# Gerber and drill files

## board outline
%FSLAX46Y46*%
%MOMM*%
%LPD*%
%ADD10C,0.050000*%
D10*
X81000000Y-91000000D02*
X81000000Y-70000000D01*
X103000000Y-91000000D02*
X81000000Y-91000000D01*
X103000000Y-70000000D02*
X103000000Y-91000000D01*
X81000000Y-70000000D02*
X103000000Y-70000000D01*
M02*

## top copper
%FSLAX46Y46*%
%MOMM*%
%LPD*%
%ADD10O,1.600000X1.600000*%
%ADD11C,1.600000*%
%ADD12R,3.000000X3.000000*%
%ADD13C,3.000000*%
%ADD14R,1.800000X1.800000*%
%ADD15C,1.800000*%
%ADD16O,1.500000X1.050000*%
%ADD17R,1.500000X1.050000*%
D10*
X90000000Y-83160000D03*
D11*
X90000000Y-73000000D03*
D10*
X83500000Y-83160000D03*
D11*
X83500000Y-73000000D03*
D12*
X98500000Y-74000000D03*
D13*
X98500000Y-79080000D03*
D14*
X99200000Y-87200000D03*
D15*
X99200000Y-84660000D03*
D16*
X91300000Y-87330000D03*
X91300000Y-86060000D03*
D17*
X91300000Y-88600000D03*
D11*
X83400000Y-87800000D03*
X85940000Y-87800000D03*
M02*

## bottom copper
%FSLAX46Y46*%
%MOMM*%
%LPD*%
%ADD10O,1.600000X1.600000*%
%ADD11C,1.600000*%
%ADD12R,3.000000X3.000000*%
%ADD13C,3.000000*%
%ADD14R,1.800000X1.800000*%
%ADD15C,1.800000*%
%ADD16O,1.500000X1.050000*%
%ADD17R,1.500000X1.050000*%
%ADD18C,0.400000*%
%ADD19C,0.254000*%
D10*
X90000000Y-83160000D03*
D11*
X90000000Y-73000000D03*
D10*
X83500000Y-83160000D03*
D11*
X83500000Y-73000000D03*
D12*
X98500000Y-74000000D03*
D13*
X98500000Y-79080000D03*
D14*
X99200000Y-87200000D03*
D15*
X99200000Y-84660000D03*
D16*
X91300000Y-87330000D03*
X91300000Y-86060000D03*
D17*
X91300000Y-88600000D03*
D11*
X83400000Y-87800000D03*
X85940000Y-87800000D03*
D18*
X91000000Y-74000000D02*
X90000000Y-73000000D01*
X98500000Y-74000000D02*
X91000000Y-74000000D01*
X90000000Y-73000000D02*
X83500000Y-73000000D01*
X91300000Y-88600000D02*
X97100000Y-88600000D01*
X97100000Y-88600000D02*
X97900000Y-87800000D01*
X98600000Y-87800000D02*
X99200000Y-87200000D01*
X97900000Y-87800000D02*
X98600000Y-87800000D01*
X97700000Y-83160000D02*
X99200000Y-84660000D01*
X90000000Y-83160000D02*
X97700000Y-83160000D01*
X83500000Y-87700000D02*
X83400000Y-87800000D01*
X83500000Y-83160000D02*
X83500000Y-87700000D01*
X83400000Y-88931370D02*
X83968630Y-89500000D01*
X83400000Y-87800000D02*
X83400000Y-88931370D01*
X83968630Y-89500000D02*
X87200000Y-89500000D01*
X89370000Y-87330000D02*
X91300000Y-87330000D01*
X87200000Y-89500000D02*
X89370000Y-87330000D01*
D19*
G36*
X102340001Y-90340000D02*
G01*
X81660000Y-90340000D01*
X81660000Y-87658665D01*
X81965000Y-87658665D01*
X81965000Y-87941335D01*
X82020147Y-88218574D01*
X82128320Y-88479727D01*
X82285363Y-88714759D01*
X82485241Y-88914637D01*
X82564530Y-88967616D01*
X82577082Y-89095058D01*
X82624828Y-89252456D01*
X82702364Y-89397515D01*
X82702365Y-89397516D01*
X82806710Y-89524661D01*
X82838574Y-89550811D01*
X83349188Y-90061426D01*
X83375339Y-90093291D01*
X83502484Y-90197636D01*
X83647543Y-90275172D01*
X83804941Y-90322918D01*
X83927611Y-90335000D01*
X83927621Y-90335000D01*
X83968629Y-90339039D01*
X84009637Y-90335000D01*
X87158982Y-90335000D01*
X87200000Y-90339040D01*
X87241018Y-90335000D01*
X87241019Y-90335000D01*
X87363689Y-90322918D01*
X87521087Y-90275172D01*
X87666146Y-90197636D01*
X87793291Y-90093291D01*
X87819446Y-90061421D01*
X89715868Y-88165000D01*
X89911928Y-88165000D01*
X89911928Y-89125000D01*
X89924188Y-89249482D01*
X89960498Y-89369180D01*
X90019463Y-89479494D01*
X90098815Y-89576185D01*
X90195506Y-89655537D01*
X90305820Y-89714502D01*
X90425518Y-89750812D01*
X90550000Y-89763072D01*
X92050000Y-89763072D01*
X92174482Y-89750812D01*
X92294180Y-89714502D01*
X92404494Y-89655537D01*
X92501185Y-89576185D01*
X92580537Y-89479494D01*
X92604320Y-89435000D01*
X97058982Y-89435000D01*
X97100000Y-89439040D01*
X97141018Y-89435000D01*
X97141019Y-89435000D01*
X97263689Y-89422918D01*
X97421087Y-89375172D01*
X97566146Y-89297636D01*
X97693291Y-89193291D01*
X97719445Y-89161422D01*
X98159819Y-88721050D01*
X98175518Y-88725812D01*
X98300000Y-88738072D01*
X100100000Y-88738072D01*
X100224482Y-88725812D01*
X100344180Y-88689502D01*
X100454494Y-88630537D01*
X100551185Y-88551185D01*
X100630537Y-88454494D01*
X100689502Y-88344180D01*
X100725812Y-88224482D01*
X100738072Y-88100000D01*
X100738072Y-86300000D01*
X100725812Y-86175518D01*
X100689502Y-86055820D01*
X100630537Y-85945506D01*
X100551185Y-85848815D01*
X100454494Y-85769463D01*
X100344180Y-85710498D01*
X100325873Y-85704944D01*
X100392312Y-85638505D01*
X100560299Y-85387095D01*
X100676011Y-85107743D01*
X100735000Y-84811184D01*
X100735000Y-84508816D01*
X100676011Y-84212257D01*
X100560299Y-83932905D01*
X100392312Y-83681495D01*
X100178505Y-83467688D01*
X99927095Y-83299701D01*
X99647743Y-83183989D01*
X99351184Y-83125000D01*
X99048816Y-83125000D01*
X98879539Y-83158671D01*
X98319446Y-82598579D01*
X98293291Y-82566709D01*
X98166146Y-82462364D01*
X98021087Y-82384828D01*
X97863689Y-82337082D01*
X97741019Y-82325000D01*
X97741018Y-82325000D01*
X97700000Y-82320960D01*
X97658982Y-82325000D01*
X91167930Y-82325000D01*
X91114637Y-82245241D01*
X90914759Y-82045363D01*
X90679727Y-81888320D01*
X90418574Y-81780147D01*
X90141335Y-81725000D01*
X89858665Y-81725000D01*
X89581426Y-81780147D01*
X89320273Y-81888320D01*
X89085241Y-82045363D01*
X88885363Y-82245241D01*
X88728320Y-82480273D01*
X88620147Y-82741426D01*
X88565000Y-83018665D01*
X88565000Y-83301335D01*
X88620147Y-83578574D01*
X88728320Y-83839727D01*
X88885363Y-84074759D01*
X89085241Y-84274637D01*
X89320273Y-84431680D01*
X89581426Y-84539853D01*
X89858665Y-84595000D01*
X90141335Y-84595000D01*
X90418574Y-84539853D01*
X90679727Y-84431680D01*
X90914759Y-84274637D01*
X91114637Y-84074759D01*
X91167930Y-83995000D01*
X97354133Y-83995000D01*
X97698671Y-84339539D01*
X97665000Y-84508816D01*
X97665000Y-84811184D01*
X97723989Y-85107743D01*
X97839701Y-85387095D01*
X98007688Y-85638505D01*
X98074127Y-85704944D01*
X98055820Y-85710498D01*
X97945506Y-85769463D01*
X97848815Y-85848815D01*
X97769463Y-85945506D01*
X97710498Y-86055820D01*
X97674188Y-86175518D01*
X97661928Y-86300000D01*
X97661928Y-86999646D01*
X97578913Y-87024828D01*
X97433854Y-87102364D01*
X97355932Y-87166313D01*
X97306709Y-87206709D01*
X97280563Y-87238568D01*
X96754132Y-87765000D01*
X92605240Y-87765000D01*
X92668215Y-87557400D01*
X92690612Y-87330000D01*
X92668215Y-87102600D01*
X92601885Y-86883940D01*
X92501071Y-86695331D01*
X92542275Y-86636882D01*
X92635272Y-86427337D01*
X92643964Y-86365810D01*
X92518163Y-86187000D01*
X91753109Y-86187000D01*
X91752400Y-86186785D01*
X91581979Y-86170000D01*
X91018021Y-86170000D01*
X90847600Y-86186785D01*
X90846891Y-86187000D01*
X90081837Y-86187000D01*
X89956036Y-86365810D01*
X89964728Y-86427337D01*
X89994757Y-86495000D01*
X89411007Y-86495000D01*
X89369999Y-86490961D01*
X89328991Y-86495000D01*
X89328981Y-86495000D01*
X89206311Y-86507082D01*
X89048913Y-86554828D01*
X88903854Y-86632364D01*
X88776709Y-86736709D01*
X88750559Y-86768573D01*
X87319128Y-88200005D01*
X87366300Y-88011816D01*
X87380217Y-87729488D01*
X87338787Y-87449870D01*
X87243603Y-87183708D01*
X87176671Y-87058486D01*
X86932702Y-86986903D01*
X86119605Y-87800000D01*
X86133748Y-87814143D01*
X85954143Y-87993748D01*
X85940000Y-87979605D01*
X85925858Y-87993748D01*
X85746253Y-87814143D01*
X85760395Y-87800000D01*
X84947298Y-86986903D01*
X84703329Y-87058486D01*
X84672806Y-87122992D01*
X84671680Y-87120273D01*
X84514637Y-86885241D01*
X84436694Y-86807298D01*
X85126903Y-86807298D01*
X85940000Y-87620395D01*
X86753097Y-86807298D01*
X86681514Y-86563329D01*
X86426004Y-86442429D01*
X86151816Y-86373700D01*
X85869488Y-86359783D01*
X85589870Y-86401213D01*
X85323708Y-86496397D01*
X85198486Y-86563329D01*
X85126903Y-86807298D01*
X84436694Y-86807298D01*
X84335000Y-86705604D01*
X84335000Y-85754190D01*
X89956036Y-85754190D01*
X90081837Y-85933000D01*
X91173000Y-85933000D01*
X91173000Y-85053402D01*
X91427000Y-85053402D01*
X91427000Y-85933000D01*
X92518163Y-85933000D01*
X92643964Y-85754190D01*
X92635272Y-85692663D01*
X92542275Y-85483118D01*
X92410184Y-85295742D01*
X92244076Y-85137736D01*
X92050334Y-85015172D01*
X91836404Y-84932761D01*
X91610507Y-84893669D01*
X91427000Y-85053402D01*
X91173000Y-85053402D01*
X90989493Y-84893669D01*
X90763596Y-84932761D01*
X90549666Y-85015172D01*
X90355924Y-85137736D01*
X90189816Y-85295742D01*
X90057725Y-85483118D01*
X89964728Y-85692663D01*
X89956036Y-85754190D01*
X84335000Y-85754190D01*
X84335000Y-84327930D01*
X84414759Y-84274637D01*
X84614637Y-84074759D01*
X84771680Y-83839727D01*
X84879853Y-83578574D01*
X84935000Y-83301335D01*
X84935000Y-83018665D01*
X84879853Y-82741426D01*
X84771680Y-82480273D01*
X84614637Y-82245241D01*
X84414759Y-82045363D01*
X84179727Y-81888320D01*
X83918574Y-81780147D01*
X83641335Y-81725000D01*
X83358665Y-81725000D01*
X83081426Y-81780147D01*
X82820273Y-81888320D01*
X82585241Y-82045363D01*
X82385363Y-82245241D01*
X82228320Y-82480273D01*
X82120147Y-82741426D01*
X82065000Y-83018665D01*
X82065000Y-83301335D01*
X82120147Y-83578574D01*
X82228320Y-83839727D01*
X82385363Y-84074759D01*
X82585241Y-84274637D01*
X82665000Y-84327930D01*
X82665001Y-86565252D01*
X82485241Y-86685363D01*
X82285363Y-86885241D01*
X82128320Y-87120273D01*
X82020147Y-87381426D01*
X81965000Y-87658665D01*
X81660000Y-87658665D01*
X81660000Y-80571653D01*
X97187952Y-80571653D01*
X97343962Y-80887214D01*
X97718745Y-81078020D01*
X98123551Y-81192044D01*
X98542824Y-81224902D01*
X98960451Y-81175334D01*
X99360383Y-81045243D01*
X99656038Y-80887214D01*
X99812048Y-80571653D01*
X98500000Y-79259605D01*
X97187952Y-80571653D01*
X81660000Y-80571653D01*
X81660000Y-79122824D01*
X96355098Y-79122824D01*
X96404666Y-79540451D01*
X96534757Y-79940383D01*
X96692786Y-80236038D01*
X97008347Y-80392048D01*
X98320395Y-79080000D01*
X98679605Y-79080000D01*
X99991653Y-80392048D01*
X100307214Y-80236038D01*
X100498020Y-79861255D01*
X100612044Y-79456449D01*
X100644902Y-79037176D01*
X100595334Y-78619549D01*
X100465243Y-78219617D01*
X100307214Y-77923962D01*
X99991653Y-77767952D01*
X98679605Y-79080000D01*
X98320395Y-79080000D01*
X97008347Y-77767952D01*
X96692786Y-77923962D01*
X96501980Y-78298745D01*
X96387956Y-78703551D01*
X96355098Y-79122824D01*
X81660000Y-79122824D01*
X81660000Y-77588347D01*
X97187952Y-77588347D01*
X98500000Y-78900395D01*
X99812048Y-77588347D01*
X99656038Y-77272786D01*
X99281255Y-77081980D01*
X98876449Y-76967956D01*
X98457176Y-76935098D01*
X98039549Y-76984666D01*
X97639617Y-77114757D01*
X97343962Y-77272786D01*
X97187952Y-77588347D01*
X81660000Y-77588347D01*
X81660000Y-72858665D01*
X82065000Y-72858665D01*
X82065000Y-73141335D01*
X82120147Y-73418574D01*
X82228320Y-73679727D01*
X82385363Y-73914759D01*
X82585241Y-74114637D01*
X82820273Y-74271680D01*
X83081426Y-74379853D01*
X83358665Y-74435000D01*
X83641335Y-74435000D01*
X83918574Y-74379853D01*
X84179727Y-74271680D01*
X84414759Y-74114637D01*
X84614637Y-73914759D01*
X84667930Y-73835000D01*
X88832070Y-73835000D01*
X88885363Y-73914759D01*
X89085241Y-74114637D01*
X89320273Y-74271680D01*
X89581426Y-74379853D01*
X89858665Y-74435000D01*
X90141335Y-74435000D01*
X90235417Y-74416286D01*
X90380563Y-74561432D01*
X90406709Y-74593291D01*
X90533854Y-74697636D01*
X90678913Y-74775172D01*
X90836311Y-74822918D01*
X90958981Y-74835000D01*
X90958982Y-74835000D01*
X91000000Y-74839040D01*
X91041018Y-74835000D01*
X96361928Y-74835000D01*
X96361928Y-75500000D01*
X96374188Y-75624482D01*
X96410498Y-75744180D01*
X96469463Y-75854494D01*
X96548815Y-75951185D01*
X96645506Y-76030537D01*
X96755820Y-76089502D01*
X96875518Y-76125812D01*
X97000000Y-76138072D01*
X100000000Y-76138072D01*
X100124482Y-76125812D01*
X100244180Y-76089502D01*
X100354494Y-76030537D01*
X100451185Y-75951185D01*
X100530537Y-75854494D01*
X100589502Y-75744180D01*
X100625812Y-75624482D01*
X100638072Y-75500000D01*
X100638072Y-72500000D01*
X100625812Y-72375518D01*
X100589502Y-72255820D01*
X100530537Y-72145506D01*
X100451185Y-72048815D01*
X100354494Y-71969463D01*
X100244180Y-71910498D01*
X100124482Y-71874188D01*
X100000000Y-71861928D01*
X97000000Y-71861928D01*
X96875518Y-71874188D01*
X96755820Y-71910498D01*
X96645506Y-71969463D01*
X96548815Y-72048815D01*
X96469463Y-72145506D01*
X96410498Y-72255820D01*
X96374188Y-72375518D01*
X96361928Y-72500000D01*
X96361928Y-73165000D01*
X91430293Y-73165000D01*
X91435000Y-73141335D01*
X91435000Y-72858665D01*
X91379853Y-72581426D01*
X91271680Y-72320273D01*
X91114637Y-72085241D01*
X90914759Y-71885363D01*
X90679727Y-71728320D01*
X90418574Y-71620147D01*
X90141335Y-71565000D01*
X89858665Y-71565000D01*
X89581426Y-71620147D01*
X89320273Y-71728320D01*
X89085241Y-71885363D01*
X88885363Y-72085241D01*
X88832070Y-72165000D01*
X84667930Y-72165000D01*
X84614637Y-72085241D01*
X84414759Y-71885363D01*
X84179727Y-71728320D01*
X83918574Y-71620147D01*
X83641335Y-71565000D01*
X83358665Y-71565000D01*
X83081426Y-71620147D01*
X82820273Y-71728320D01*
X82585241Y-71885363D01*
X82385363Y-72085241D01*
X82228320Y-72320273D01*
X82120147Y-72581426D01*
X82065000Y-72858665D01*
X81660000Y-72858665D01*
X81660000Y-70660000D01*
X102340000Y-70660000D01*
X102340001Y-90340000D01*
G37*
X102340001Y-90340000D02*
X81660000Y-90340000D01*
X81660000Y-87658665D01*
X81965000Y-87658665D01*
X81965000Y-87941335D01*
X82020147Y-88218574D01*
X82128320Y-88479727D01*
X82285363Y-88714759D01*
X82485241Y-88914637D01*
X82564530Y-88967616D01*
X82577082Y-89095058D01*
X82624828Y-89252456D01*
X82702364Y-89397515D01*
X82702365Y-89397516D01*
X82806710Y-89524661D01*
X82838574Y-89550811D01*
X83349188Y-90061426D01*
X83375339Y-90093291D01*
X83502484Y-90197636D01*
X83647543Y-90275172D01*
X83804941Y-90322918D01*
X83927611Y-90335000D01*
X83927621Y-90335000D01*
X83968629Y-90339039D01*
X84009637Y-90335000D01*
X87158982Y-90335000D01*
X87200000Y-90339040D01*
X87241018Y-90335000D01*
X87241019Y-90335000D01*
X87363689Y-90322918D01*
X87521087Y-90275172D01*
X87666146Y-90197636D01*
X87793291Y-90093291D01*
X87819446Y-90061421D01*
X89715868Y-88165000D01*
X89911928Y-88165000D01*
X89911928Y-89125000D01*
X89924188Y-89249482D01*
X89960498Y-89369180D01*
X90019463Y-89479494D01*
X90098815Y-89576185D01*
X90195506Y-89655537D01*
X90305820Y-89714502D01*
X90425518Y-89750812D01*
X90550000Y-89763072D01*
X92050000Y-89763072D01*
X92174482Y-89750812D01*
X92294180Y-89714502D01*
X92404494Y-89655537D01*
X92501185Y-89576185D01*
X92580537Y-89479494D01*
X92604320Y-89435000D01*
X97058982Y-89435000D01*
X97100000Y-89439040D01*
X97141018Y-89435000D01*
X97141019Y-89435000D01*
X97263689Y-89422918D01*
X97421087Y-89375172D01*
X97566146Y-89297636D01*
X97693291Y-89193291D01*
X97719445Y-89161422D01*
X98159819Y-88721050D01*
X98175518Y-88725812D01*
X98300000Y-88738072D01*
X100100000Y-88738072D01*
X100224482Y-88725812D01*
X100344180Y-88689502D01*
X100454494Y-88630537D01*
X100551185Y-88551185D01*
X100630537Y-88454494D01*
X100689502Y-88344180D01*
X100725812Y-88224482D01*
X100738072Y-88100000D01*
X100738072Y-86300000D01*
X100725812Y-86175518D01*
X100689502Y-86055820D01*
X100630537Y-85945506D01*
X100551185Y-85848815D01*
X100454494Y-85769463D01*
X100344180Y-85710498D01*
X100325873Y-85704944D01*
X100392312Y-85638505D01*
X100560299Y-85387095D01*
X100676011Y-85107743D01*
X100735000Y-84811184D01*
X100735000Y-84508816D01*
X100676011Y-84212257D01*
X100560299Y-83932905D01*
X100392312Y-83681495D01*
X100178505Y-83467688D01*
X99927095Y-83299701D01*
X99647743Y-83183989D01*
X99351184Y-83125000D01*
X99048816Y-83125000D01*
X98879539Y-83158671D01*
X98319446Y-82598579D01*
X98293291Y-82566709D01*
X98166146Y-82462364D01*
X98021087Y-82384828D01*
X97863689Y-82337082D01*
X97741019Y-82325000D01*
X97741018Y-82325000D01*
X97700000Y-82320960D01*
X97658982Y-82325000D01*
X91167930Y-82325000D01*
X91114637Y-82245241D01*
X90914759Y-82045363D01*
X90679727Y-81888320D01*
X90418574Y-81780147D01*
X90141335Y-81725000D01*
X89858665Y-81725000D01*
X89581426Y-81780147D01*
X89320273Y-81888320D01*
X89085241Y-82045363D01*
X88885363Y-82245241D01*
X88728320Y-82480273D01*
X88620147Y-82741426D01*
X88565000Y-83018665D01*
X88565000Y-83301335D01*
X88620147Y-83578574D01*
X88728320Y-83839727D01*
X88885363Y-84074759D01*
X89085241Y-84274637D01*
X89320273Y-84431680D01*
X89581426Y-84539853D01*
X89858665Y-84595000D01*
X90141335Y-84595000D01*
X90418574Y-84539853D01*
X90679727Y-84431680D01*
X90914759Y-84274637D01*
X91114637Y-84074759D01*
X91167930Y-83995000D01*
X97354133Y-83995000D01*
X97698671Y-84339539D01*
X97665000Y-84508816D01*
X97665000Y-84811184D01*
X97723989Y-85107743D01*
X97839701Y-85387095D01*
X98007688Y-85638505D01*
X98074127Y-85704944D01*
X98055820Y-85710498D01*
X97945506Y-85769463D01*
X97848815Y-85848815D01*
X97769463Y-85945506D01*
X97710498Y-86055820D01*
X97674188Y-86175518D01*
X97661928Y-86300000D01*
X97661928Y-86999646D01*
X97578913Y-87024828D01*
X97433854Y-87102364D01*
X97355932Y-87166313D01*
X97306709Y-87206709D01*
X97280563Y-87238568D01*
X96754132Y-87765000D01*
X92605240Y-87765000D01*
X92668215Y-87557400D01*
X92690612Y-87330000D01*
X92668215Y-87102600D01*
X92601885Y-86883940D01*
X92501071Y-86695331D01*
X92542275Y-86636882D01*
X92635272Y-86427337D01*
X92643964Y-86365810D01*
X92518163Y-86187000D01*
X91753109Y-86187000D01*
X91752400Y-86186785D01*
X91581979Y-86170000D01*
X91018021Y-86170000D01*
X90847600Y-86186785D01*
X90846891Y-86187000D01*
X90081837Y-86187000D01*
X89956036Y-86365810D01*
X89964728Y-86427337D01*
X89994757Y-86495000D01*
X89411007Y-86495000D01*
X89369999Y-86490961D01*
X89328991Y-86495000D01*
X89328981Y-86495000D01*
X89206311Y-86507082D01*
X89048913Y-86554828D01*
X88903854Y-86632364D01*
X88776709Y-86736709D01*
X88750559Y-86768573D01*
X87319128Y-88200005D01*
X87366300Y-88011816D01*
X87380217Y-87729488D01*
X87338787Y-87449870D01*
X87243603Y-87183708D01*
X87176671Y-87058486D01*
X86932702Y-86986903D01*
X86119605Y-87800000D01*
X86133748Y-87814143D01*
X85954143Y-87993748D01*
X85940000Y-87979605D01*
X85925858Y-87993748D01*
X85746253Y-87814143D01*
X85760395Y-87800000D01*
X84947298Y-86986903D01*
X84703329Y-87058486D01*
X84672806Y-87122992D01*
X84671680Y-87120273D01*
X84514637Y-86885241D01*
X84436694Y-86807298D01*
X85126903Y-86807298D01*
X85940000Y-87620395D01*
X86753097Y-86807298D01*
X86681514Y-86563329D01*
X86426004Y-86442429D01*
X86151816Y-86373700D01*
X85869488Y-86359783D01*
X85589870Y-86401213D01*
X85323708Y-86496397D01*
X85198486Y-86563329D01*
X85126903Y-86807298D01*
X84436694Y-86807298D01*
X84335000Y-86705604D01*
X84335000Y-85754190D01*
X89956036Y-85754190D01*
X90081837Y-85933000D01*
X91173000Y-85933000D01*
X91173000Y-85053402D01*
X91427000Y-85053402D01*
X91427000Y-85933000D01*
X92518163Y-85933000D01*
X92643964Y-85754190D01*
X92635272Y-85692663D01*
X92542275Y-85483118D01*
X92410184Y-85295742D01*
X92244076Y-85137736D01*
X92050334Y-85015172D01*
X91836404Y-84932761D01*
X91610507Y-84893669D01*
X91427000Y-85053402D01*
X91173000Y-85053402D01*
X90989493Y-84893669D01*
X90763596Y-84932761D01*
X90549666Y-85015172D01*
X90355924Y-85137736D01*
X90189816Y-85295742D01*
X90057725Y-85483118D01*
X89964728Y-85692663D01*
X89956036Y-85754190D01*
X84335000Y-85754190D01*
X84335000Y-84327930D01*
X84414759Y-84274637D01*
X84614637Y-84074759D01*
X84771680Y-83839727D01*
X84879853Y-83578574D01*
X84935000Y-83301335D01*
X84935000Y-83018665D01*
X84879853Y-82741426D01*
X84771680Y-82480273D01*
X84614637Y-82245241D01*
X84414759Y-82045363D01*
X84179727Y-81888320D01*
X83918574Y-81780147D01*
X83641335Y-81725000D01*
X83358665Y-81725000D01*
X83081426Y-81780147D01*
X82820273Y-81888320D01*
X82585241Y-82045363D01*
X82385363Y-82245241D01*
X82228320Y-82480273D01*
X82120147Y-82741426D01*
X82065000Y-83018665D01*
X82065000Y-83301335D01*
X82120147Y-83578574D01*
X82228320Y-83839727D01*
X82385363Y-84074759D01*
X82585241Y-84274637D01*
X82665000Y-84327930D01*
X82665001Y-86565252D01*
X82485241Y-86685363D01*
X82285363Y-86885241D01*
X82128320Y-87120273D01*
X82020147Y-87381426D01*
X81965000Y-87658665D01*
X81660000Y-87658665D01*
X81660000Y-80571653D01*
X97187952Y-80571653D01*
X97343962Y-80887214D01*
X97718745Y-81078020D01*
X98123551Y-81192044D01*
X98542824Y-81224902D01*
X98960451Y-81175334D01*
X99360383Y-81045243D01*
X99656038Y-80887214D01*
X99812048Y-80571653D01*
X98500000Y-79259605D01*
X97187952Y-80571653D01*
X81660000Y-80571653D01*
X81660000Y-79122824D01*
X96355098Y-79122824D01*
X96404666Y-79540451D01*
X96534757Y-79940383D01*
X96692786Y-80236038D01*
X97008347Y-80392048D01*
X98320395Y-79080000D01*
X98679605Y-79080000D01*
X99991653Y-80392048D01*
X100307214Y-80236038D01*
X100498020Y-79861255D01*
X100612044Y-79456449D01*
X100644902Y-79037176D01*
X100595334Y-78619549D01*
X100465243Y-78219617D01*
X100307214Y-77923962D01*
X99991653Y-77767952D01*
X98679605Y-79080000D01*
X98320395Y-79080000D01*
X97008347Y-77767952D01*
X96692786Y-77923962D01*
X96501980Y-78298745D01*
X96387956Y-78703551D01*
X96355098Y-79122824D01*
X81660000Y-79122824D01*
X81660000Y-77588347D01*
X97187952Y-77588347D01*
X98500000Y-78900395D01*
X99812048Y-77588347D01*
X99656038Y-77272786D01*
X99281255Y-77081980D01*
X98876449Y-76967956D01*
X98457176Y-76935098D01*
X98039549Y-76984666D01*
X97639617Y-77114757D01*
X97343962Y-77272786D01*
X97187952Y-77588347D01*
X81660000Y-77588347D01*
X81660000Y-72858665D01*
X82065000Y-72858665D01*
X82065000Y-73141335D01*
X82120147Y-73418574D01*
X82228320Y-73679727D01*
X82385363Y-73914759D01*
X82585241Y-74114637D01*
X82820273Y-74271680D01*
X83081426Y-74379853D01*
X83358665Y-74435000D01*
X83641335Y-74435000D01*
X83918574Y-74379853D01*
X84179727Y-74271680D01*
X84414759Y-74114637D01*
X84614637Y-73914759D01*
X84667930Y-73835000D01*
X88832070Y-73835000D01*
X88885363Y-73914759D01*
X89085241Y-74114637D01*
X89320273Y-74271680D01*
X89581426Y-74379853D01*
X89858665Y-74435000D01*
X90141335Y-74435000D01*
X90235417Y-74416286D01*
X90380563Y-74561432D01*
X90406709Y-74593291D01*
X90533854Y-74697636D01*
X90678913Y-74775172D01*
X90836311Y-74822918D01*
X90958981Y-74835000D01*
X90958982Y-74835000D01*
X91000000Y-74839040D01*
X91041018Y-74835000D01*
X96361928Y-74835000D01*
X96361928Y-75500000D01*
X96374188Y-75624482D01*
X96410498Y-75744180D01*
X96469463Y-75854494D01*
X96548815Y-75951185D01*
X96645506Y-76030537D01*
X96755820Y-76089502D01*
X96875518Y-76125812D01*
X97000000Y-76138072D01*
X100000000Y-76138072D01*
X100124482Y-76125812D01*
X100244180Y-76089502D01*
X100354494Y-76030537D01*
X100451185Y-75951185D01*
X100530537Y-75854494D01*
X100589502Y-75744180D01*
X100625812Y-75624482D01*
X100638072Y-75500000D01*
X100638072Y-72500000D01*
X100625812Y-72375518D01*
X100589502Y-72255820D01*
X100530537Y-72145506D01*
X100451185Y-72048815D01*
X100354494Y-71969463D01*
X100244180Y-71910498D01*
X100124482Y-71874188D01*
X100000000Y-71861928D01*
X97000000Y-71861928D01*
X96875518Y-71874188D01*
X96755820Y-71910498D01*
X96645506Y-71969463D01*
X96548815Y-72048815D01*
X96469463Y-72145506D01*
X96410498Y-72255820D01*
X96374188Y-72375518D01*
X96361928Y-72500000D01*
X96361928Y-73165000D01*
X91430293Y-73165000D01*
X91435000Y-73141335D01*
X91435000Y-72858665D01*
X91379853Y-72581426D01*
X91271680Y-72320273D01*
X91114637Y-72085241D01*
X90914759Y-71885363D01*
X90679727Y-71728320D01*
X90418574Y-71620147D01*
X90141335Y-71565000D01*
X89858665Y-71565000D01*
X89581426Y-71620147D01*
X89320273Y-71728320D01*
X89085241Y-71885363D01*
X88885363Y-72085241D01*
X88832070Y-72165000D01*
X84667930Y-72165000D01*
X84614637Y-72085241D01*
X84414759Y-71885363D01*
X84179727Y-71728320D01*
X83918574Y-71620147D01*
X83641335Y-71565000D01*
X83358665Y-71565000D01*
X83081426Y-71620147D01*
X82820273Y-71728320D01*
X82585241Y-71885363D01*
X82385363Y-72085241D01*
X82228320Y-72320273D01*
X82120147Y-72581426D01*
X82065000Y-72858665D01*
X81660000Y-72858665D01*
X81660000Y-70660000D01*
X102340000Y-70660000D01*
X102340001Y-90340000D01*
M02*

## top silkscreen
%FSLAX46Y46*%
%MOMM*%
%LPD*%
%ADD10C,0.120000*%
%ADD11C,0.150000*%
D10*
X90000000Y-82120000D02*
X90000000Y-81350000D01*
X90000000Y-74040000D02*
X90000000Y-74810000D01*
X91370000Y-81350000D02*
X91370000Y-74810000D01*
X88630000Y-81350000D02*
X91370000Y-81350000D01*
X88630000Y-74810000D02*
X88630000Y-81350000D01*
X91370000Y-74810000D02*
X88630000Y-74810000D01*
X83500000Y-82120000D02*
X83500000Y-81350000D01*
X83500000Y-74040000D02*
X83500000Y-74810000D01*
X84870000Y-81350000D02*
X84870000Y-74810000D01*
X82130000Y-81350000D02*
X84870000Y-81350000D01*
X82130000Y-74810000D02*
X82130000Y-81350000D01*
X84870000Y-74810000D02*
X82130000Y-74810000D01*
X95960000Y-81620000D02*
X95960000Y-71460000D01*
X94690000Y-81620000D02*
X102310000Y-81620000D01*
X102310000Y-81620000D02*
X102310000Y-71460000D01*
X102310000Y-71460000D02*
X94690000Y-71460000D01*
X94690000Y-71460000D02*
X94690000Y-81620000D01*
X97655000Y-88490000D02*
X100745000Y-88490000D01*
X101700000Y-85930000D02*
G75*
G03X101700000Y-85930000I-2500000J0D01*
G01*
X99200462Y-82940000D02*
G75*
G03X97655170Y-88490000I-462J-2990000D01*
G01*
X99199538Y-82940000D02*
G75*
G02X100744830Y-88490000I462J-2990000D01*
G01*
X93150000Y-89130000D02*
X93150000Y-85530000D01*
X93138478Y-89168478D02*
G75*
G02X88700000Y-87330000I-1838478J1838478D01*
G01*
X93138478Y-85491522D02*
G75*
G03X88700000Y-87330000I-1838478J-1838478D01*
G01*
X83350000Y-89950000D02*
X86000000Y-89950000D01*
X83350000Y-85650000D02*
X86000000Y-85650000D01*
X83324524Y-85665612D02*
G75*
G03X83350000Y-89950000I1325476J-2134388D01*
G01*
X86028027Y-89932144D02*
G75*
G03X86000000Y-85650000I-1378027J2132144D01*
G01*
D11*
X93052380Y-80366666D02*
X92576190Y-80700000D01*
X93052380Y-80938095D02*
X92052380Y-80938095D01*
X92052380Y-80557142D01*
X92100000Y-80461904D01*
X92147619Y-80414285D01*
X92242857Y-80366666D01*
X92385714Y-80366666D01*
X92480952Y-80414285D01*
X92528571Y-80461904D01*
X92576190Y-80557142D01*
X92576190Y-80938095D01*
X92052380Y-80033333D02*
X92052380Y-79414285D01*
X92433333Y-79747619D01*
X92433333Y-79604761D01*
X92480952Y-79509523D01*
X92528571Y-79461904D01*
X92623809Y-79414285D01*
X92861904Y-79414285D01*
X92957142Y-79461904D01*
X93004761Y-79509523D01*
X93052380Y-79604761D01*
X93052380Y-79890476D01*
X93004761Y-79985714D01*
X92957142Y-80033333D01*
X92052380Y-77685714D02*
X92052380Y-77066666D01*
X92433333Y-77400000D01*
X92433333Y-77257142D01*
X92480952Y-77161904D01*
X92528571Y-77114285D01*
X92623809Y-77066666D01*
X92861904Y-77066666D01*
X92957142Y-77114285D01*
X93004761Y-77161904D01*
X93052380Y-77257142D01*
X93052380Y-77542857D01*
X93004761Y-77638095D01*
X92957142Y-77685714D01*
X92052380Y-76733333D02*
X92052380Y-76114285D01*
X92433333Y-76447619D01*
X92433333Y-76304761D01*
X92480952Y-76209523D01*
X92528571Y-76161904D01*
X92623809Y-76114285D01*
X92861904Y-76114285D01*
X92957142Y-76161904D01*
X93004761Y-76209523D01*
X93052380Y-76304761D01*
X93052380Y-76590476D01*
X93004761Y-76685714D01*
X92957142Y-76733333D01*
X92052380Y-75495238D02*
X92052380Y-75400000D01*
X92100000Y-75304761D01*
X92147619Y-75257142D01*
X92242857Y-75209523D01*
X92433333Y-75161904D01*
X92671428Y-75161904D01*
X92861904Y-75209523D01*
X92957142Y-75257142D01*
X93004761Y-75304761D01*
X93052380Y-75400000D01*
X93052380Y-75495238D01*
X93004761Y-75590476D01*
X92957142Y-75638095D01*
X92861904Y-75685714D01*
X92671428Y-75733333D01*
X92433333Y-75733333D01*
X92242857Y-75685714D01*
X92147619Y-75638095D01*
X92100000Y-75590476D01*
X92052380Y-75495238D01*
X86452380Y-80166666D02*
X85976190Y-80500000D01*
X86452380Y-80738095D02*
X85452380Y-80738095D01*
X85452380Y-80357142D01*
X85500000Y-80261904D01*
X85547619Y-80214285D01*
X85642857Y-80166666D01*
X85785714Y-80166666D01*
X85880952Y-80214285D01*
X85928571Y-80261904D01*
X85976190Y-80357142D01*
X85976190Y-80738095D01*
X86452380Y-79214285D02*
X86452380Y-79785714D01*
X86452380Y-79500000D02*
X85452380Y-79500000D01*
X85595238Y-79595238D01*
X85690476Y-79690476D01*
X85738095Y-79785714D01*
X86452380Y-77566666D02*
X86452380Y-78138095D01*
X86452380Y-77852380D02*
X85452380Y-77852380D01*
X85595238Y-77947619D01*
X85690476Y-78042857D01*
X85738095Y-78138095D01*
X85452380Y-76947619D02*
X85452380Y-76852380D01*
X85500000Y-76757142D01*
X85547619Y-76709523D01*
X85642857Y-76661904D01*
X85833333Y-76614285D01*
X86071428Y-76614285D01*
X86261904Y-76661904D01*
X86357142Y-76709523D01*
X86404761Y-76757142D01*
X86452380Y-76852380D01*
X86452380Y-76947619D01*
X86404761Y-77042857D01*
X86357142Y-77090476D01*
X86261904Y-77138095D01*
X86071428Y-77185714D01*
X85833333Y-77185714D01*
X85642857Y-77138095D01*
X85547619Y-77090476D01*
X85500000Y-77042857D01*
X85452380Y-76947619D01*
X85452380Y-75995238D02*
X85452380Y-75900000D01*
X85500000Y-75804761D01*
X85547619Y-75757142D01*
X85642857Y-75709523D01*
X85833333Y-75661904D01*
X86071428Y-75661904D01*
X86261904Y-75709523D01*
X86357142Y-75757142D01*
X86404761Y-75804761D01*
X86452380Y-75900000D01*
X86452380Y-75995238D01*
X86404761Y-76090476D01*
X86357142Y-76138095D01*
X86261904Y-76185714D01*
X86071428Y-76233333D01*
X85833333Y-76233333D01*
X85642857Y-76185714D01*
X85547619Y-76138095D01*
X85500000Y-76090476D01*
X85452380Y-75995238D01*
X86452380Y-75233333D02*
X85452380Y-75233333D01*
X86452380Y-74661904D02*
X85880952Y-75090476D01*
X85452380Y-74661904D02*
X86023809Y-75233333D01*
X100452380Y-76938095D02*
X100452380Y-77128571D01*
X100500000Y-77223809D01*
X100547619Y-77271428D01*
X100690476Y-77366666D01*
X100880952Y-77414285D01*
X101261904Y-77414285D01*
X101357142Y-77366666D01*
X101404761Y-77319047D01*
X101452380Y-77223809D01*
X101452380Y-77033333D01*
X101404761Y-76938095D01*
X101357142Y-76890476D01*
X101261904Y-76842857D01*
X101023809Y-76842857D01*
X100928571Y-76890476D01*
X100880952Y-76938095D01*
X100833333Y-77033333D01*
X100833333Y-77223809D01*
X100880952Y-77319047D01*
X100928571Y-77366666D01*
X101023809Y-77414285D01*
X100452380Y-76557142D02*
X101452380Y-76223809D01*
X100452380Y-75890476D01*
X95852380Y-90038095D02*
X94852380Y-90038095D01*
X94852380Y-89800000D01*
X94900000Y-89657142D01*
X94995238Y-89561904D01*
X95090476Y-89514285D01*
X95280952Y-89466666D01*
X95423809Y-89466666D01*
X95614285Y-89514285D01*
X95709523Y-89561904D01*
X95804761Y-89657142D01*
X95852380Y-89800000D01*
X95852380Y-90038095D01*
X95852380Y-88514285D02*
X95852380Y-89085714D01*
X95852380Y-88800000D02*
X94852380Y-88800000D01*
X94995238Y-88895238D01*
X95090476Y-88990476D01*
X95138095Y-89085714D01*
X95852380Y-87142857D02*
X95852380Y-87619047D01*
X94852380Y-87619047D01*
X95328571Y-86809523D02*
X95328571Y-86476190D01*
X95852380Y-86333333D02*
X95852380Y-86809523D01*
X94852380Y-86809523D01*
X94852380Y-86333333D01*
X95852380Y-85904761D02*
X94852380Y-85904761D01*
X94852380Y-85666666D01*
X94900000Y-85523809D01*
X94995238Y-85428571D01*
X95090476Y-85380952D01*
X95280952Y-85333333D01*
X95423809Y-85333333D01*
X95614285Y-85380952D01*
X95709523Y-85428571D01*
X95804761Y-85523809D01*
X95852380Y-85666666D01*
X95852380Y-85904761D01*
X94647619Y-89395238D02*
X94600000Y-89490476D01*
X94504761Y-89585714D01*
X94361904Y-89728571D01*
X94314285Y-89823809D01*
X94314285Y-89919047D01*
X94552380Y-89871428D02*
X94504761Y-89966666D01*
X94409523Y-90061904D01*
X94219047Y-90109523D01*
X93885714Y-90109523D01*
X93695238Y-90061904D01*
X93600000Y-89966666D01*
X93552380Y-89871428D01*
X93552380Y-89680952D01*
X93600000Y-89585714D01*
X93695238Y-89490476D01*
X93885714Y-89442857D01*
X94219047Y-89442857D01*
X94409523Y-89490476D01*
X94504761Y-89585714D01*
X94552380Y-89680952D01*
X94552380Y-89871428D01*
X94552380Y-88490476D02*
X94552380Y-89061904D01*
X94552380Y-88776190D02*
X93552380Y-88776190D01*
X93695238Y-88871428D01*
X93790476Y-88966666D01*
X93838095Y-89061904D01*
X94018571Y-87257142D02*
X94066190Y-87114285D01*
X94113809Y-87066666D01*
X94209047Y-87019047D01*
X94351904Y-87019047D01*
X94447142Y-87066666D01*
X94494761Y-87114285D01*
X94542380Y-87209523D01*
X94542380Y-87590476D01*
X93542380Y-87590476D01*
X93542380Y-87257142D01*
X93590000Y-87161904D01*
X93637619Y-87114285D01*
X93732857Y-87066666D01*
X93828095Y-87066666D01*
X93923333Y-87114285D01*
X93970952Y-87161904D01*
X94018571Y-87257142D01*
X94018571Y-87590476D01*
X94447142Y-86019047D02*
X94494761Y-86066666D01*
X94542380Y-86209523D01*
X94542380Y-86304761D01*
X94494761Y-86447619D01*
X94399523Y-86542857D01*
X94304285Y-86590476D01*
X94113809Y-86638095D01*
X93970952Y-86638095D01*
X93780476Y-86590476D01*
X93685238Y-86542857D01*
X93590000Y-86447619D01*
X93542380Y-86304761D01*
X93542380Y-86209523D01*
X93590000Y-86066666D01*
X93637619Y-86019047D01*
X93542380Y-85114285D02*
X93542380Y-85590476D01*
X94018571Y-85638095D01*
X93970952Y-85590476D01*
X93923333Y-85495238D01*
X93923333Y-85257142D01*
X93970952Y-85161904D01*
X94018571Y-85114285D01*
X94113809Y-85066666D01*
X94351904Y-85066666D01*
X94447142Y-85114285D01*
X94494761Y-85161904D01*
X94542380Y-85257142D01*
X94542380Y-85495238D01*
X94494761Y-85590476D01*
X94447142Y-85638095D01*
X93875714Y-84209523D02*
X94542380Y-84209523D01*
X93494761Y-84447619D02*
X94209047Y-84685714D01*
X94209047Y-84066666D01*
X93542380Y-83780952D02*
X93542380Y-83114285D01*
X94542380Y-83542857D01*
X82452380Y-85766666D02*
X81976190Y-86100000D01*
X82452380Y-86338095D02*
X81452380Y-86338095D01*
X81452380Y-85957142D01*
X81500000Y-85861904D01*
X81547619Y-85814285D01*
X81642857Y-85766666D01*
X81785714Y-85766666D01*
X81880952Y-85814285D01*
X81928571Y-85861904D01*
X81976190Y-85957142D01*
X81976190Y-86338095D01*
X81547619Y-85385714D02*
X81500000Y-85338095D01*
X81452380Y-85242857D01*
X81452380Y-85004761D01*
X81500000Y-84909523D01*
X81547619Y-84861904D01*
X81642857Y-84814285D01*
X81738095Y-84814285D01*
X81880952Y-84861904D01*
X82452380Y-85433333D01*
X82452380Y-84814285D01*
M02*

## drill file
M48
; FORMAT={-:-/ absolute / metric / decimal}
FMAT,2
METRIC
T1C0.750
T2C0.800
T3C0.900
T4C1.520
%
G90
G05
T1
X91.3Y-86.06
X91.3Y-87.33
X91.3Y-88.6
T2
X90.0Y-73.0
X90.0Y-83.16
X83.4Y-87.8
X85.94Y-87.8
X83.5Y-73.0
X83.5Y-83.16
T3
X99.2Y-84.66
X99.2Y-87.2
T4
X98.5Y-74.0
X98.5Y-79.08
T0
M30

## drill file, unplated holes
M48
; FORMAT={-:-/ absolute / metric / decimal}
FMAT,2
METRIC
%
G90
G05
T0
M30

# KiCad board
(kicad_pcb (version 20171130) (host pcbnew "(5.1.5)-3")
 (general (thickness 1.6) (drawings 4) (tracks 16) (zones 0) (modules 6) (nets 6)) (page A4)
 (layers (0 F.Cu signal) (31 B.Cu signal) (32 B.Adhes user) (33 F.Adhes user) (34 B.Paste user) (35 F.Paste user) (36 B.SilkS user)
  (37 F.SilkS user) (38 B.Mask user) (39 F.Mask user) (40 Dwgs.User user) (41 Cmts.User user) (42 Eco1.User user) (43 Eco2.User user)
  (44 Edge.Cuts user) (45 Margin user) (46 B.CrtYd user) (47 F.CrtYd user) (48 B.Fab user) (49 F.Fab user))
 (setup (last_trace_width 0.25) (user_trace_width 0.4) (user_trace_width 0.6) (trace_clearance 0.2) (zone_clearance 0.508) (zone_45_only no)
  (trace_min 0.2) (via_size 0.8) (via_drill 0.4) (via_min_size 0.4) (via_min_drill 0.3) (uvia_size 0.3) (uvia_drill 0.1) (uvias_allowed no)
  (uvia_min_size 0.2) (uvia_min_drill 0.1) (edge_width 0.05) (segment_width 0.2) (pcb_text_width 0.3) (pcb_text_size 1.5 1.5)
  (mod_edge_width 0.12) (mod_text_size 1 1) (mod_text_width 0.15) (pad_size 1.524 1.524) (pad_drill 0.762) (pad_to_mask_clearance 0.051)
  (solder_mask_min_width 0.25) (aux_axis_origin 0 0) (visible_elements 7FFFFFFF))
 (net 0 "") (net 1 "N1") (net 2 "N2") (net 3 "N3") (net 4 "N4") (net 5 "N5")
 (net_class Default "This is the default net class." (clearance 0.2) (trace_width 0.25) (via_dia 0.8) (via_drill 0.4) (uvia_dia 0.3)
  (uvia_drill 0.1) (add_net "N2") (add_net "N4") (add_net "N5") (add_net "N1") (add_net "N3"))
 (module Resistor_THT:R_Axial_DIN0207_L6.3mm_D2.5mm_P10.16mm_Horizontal (layer F.Cu) (at 90 73 270)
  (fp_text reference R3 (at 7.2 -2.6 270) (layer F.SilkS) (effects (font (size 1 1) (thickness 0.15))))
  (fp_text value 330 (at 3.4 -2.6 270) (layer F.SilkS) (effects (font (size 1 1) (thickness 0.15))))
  (fp_line (start 9.12 0) (end 8.35 0) (layer F.SilkS) (width 0.12))
  (fp_line (start 1.04 0) (end 1.81 0) (layer F.SilkS) (width 0.12))
  (fp_line (start 8.35 -1.37) (end 1.81 -1.37) (layer F.SilkS) (width 0.12))
  (fp_line (start 8.35 1.37) (end 8.35 -1.37) (layer F.SilkS) (width 0.12))
  (fp_line (start 1.81 1.37) (end 8.35 1.37) (layer F.SilkS) (width 0.12))
  (fp_line (start 1.81 -1.37) (end 1.81 1.37) (layer F.SilkS) (width 0.12))
  (pad 2 thru_hole oval (at 10.16 0 270) (size 1.6 1.6) (drill 0.8) (layers *.Cu *.Mask) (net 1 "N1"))
  (pad 1 thru_hole circle (at 0 0 270) (size 1.6 1.6) (drill 0.8) (layers *.Cu *.Mask) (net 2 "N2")))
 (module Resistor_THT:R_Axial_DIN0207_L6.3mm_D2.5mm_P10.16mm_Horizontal (layer F.Cu) (at 83.5 73 270)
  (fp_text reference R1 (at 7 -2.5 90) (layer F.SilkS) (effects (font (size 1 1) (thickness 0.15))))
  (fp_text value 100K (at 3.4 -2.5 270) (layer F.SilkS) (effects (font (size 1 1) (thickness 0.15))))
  (fp_line (start 9.12 0) (end 8.35 0) (layer F.SilkS) (width 0.12))
  (fp_line (start 1.04 0) (end 1.81 0) (layer F.SilkS) (width 0.12))
  (fp_line (start 8.35 -1.37) (end 1.81 -1.37) (layer F.SilkS) (width 0.12))
  (fp_line (start 8.35 1.37) (end 8.35 -1.37) (layer F.SilkS) (width 0.12))
  (fp_line (start 1.81 1.37) (end 8.35 1.37) (layer F.SilkS) (width 0.12))
  (fp_line (start 1.81 -1.37) (end 1.81 1.37) (layer F.SilkS) (width 0.12))
  (pad 2 thru_hole oval (at 10.16 0 270) (size 1.6 1.6) (drill 0.8) (layers *.Cu *.Mask) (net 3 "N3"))
  (pad 1 thru_hole circle (at 0 0 270) (size 1.6 1.6) (drill 0.8) (layers *.Cu *.Mask) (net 2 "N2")))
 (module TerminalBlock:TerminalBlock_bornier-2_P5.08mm (layer F.Cu) (at 98.5 74 270)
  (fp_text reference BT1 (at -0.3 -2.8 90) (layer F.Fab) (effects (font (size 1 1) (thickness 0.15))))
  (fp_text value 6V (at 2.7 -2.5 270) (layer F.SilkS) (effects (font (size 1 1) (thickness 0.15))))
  (fp_line (start 7.62 2.54) (end -2.54 2.54) (layer F.SilkS) (width 0.12))
  (fp_line (start 7.62 3.81) (end 7.62 -3.81) (layer F.SilkS) (width 0.12))
  (fp_line (start 7.62 -3.81) (end -2.54 -3.81) (layer F.SilkS) (width 0.12))
  (fp_line (start -2.54 -3.81) (end -2.54 3.81) (layer F.SilkS) (width 0.12))
  (fp_line (start -2.54 3.81) (end 7.62 3.81) (layer F.SilkS) (width 0.12))
  (pad 1 thru_hole rect (at 0 0 270) (size 3 3) (drill 1.52) (layers *.Cu *.Mask) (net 2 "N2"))
  (pad 2 thru_hole circle (at 5.08 0 270) (size 3 3) (drill 1.52) (layers *.Cu *.Mask) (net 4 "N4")))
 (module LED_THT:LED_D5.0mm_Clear (layer F.Cu) (at 99.2 87.2 90)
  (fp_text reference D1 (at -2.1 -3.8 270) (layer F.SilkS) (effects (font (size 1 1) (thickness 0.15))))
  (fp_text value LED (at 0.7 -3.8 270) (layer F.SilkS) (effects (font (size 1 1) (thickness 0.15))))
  (fp_line (start -1.29 -1.545) (end -1.29 1.545) (layer F.SilkS) (width 0.12))
  (fp_circle (center 1.27 0) (end 3.77 0) (layer F.SilkS) (width 0.12))
  (fp_arc (start 1.27 0) (end -1.29 -1.54483) (angle 148.9) (layer F.SilkS) (width 0.12))
  (fp_arc (start 1.27 0) (end -1.29 1.54483) (angle -148.9) (layer F.SilkS) (width 0.12))
  (pad 1 thru_hole rect (at 0 0 90) (size 1.8 1.8) (drill 0.9) (layers *.Cu *.Mask) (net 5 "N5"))
  (pad 2 thru_hole circle (at 2.54 0 90) (size 1.8 1.8) (drill 0.9) (layers *.Cu *.Mask) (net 1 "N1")))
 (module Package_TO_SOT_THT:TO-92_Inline (layer F.Cu) (at 91.3 88.6 90)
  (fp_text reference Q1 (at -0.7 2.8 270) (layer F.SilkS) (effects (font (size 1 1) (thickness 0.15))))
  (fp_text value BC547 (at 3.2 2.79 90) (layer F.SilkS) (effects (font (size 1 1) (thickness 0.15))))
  (fp_line (start -0.53 1.85) (end 3.07 1.85) (layer F.SilkS) (width 0.12))
  (fp_arc (start 1.27 0) (end 1.27 -2.6) (angle -135) (layer F.SilkS) (width 0.12))
  (fp_arc (start 1.27 0) (end 1.27 -2.6) (angle 135) (layer F.SilkS) (width 0.12))
  (pad 2 thru_hole oval (at 1.27 0 90) (size 1.05 1.5) (drill 0.75) (layers *.Cu *.Mask) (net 3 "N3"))
  (pad 3 thru_hole oval (at 2.54 0 90) (size 1.05 1.5) (drill 0.75) (layers *.Cu *.Mask) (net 4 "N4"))
  (pad 1 thru_hole rect (at 0 0 90) (size 1.05 1.5) (drill 0.75) (layers *.Cu *.Mask) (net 5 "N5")))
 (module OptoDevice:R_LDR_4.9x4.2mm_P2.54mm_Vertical (layer F.Cu) (at 83.4 87.8)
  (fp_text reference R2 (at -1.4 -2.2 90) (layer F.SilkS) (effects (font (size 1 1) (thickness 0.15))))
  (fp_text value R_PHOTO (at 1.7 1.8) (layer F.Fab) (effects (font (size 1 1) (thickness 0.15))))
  (fp_line (start -0.05 2.15) (end 2.6 2.15) (layer F.SilkS) (width 0.12))
  (fp_line (start -0.05 -2.15) (end 2.6 -2.15) (layer F.SilkS) (width 0.12))
  (fp_arc (start 1.25 0) (end -0.05 2.15) (angle 117) (layer F.SilkS) (width 0.12))
  (fp_arc (start 1.25 0) (end 2.6 -2.15) (angle 115) (layer F.SilkS) (width 0.12))
  (pad 1 thru_hole circle (at 0 0) (size 1.6 1.6) (drill 0.8) (layers *.Cu *.Mask) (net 3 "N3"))
  (pad 2 thru_hole circle (at 2.54 0) (size 1.6 1.6) (drill 0.8) (layers *.Cu *.Mask) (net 4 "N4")))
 (gr_line (start 81 91) (end 81 70) (layer Edge.Cuts) (width 0.05))
 (gr_line (start 103 91) (end 81 91) (layer Edge.Cuts) (width 0.05))
 (gr_line (start 103 70) (end 103 91) (layer Edge.Cuts) (width 0.05))
 (gr_line (start 81 70) (end 103 70) (layer Edge.Cuts) (width 0.05))
 (segment (start 91 74) (end 90 73) (width 0.4) (layer B.Cu) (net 2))
 (segment (start 98.5 74) (end 91 74) (width 0.4) (layer B.Cu) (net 2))
 (segment (start 90 73) (end 83.5 73) (width 0.4) (layer B.Cu) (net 2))
 (segment (start 91.3 88.6) (end 97.1 88.6) (width 0.4) (layer B.Cu) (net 5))
 (segment (start 97.1 88.6) (end 97.9 87.8) (width 0.4) (layer B.Cu) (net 5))
 (segment (start 98.6 87.8) (end 99.2 87.2) (width 0.4) (layer B.Cu) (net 5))
 (segment (start 97.9 87.8) (end 98.6 87.8) (width 0.4) (layer B.Cu) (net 5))
 (segment (start 97.7 83.16) (end 99.2 84.66) (width 0.4) (layer B.Cu) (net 1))
 (segment (start 90 83.16) (end 97.7 83.16) (width 0.4) (layer B.Cu) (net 1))
 (segment (start 83.5 87.7) (end 83.4 87.8) (width 0.4) (layer B.Cu) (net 3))
 (segment (start 83.5 83.16) (end 83.5 87.7) (width 0.4) (layer B.Cu) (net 3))
 (segment (start 83.4 88.93137) (end 83.96863 89.5) (width 0.4) (layer B.Cu) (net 3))
 (segment (start 83.4 87.8) (end 83.4 88.93137) (width 0.4) (layer B.Cu) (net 3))
 (segment (start 83.96863 89.5) (end 87.2 89.5) (width 0.4) (layer B.Cu) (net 3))
 (segment (start 89.37 87.33) (end 91.3 87.33) (width 0.4) (layer B.Cu) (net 3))
 (segment (start 87.2 89.5) (end 89.37 87.33) (width 0.4) (layer B.Cu) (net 3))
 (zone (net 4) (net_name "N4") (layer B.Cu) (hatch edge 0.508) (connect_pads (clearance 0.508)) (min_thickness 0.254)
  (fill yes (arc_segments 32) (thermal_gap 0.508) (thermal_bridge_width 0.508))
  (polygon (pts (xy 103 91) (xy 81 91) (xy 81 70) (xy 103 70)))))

